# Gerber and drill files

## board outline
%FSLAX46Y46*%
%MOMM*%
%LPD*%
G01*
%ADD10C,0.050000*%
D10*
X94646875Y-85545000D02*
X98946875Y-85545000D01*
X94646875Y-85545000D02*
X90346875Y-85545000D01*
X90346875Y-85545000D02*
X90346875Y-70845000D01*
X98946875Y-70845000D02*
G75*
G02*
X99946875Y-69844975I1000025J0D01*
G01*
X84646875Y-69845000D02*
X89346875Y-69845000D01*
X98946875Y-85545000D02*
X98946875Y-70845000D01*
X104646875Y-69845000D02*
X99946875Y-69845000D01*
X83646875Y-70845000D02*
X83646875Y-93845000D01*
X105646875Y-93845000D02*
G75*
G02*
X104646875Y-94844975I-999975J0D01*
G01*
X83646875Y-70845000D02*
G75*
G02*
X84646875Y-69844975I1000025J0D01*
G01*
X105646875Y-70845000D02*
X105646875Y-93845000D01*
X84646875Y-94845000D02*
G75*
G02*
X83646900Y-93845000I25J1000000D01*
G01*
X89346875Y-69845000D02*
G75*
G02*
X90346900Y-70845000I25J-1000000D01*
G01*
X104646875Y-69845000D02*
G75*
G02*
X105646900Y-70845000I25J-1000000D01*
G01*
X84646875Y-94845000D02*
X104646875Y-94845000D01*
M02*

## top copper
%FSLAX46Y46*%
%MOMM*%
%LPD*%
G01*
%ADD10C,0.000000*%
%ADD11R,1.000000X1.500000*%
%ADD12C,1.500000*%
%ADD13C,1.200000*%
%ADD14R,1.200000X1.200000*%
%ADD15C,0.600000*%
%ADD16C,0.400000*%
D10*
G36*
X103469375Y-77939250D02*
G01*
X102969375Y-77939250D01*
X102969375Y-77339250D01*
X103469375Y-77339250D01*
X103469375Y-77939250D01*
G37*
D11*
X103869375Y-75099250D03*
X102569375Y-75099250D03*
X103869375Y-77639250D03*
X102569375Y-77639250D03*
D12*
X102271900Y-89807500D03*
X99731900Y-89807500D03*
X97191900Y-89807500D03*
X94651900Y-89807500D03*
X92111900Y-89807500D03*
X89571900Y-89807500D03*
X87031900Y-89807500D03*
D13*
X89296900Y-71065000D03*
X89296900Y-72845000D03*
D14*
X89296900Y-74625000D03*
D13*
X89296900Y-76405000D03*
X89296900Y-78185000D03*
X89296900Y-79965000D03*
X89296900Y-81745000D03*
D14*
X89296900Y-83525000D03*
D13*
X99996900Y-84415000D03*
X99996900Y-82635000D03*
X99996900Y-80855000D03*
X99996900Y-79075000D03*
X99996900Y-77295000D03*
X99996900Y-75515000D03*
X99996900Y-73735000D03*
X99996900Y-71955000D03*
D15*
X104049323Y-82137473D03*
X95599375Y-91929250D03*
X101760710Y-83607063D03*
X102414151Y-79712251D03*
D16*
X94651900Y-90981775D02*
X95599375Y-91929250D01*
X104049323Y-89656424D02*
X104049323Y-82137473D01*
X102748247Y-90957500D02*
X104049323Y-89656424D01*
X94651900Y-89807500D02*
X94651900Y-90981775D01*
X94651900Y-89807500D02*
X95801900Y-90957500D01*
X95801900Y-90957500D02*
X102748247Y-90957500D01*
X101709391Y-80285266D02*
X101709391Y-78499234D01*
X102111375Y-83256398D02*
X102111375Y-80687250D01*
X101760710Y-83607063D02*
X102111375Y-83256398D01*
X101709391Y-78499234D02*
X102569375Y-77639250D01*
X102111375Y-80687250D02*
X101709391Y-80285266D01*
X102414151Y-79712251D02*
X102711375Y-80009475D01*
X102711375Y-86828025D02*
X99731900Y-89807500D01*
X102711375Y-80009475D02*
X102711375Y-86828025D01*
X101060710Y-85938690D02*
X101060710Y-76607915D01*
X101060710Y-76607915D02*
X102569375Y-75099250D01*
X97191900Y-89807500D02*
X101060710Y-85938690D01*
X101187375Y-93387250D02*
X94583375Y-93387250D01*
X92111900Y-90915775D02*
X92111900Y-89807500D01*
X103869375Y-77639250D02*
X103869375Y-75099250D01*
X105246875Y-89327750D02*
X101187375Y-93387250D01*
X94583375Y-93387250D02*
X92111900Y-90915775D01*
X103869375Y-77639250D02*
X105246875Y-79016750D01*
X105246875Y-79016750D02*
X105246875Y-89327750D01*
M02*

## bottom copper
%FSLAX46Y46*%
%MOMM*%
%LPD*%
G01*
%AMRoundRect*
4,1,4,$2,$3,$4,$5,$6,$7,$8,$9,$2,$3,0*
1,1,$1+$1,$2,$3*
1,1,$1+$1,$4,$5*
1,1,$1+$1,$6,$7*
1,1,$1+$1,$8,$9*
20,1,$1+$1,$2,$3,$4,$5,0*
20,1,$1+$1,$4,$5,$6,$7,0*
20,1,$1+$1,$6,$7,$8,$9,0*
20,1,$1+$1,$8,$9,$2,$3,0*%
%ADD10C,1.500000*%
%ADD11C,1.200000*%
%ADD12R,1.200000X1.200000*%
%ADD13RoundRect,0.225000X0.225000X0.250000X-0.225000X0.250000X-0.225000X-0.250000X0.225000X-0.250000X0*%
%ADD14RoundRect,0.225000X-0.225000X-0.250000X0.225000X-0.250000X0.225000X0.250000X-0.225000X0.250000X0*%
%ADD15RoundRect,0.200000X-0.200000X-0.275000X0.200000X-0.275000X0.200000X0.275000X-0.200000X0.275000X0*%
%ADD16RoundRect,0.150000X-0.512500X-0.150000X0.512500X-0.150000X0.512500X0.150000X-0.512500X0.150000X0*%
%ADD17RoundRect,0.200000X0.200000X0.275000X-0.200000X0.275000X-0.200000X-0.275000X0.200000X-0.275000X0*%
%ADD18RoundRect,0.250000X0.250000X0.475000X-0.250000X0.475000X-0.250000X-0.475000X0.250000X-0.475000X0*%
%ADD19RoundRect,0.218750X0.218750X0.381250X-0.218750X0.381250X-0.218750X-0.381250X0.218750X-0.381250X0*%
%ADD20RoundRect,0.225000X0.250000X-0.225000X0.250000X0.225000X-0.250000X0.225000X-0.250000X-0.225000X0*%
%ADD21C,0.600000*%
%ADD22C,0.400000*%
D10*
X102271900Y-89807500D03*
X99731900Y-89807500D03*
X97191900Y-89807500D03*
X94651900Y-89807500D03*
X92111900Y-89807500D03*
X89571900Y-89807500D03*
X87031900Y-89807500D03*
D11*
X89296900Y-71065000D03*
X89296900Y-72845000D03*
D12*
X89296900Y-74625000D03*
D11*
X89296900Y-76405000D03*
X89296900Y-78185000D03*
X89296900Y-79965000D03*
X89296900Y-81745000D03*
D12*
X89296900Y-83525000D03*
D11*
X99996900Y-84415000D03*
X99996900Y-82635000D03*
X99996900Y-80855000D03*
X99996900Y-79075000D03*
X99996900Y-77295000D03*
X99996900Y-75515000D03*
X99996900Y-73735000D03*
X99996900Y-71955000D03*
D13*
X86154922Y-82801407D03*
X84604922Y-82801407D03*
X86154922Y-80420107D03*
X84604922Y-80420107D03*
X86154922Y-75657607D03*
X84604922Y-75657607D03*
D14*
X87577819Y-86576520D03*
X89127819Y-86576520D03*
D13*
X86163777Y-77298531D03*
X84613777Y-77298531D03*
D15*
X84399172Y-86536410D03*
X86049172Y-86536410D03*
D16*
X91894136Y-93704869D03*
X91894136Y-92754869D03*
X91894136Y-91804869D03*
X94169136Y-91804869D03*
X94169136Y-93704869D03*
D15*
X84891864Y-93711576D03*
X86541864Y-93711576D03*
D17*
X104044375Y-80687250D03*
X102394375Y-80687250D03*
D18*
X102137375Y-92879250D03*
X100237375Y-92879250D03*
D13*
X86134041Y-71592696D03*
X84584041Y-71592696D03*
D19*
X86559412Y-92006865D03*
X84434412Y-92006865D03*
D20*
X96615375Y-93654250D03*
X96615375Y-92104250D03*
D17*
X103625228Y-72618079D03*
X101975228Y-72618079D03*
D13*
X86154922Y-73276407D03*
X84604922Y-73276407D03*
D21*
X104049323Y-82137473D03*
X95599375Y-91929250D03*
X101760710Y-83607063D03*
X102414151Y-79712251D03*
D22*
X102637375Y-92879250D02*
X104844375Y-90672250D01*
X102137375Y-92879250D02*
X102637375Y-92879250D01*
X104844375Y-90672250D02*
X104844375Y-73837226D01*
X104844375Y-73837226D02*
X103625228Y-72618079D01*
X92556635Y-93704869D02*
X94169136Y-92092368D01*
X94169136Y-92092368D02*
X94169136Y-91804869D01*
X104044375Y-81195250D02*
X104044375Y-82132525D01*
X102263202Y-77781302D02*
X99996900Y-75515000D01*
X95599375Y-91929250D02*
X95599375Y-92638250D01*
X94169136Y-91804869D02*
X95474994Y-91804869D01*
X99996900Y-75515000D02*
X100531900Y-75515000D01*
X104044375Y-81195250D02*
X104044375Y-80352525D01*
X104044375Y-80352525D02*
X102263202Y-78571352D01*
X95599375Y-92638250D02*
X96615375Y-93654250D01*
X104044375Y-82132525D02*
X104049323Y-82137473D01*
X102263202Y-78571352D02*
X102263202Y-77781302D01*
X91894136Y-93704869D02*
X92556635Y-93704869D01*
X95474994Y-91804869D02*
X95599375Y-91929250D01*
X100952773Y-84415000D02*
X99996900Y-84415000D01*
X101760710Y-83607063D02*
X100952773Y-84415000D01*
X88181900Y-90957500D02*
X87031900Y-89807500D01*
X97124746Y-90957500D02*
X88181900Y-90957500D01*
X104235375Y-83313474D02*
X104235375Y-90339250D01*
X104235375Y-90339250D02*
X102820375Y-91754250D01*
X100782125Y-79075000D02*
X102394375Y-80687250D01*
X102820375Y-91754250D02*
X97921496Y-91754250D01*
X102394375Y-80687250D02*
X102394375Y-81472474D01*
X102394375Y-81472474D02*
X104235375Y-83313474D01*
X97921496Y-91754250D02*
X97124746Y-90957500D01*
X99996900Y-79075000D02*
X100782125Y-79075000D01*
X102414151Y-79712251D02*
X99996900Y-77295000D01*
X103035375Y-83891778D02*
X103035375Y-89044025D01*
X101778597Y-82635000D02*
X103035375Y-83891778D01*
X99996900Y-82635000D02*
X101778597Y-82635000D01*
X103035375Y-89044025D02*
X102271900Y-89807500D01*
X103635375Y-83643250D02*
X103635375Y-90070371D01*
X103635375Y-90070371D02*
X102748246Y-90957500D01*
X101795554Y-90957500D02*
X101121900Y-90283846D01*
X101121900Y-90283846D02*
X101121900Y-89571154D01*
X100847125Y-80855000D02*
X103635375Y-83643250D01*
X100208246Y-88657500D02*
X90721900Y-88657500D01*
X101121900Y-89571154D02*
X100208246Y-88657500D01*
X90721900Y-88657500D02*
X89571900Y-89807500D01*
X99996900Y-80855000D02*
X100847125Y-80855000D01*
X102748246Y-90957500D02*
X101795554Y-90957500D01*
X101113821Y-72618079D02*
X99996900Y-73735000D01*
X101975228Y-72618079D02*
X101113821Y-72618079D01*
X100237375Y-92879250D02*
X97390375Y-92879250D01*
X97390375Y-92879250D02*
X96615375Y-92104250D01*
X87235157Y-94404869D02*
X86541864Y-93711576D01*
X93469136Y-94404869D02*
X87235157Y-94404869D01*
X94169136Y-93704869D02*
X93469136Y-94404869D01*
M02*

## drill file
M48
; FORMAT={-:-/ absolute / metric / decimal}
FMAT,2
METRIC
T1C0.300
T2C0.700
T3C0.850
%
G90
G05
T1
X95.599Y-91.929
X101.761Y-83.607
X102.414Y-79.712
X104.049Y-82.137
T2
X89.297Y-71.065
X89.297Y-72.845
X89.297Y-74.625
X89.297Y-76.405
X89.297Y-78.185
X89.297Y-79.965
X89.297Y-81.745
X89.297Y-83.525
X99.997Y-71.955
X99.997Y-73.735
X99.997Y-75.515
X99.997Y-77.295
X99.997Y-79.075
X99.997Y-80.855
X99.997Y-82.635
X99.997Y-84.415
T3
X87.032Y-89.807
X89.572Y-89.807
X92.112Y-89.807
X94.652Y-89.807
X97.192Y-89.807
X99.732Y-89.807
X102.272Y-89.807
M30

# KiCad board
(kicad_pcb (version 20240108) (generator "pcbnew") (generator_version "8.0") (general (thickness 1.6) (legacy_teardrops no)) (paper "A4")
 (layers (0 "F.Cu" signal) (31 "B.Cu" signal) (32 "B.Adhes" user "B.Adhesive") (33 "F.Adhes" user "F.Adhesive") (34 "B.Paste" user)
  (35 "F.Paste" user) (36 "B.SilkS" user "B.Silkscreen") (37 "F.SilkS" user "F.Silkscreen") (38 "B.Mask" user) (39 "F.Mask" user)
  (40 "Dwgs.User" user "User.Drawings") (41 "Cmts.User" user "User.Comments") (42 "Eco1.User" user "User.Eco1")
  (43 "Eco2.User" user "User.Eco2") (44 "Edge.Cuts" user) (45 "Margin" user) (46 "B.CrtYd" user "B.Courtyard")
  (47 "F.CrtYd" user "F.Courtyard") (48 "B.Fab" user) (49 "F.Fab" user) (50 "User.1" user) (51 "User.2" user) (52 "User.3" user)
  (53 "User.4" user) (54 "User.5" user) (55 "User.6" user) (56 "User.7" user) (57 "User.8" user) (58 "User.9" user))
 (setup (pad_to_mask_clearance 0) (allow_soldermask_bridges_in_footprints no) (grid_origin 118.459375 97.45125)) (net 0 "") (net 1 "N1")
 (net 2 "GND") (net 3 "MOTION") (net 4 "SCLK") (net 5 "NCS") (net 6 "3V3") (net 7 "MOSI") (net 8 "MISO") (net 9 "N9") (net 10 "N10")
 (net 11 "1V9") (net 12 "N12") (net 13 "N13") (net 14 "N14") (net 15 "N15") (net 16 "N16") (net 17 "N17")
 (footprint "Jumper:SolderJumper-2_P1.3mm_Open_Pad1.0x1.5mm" (layer "F.Cu") (at 103.219375 75.09925 180)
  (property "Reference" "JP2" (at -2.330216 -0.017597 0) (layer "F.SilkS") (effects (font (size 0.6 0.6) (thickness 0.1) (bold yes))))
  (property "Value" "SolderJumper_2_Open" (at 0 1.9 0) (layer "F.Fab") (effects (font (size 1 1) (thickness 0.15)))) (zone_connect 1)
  (pad "1" smd rect (at -0.65 0 180) (size 1 1.5) (layers "F.Cu" "F.Mask") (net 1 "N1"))
  (pad "2" smd rect (at 0.65 0 180) (size 1 1.5) (layers "F.Cu" "F.Mask") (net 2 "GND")))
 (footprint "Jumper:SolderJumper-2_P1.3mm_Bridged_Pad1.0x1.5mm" (layer "F.Cu") (at 103.219375 77.63925 180)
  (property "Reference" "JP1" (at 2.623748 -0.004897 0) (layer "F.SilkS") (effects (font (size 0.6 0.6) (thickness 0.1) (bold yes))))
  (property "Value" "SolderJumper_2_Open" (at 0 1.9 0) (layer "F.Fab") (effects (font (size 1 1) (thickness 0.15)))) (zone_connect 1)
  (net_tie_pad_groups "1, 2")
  (fp_poly (pts (xy -0.25 -0.3) (xy 0.25 -0.3) (xy 0.25 0.3) (xy -0.25 0.3)) (stroke (width 0) (type solid)) (fill solid) (layer "F.Cu"))
  (pad "1" smd rect (at -0.65 0 180) (size 1 1.5) (layers "F.Cu" "F.Mask") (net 1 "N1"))
  (pad "2" smd rect (at 0.65 0 180) (size 1 1.5) (layers "F.Cu" "F.Mask") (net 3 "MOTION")))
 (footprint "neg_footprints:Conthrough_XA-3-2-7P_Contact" (layer "F.Cu") (at 102.2719 89.8075 -90)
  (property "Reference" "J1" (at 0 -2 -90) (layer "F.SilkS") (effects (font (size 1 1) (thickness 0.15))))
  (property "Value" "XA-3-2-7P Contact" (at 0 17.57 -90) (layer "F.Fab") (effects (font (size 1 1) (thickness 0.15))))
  (pad "1" thru_hole circle (at 0 0 270) (size 1.5 1.5) (drill 0.85) (layers "*.Cu" "*.Mask") (remove_unused_layers no) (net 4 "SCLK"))
  (pad "2" thru_hole circle (at 0 2.54 270) (size 1.5 1.5) (drill 0.85) (layers "*.Cu" "*.Mask") (remove_unused_layers no) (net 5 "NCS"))
  (pad "3" thru_hole circle (at 0 5.08 270) (size 1.5 1.5) (drill 0.85) (layers "*.Cu" "*.Mask") (remove_unused_layers no) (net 2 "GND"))
  (pad "4" thru_hole circle (at 0 7.62 270) (size 1.5 1.5) (drill 0.85) (layers "*.Cu" "*.Mask") (remove_unused_layers no) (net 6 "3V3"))
  (pad "5" thru_hole circle (at 0 10.16 270) (size 1.5 1.5) (drill 0.85) (layers "*.Cu" "*.Mask") (remove_unused_layers no) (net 1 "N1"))
  (pad "6" thru_hole circle (at 0 12.7 270) (size 1.5 1.5) (drill 0.85) (layers "*.Cu" "*.Mask") (remove_unused_layers no) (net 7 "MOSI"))
  (pad "7" thru_hole circle (at 0 15.24 270) (size 1.5 1.5) (drill 0.85) (layers "*.Cu" "*.Mask") (remove_unused_layers no) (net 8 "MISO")))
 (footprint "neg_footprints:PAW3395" (layer "F.Cu") (at 94.6469 76.405)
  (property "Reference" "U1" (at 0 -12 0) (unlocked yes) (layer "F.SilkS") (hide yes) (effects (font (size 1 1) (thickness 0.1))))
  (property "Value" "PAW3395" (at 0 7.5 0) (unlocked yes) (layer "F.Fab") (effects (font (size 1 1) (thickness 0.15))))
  (pad "1" thru_hole circle (at -5.35 -5.34) (size 1.2 1.2) (drill 0.7) (layers "*.Cu" "*.Mask") (remove_unused_layers no) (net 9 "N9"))
  (pad "2" thru_hole circle (at -5.35 -3.56) (size 1.2 1.2) (drill 0.7) (layers "*.Cu" "*.Mask") (remove_unused_layers no) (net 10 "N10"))
  (pad "3" thru_hole rect (at -5.35 -1.78) (size 1.2 1.2) (drill 0.7) (layers "*.Cu" "*.Mask") (remove_unused_layers no) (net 2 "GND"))
  (pad "4" thru_hole circle (at -5.35 0) (size 1.2 1.2) (drill 0.7) (layers "*.Cu" "*.Mask") (remove_unused_layers no) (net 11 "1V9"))
  (pad "5" thru_hole circle (at -5.35 1.78) (size 1.2 1.2) (drill 0.7) (layers "*.Cu" "*.Mask") (remove_unused_layers no) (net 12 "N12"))
  (pad "6" thru_hole circle (at -5.35 3.56) (size 1.2 1.2) (drill 0.7) (layers "*.Cu" "*.Mask") (remove_unused_layers no) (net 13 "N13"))
  (pad "7" thru_hole circle (at -5.35 5.34) (size 1.2 1.2) (drill 0.7) (layers "*.Cu" "*.Mask") (remove_unused_layers no) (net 6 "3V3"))
  (pad "8" thru_hole rect (at -5.35 7.12) (size 1.2 1.2) (drill 0.7) (layers "*.Cu" "*.Mask") (remove_unused_layers no) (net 2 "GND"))
  (pad "9" thru_hole circle (at 5.35 8.01) (size 1.2 1.2) (drill 0.7) (layers "*.Cu" "*.Mask") (remove_unused_layers no) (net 3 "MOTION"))
  (pad "10" thru_hole circle (at 5.35 6.23) (size 1.2 1.2) (drill 0.7) (layers "*.Cu" "*.Mask") (remove_unused_layers no) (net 4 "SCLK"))
  (pad "11" thru_hole circle (at 5.35 4.45) (size 1.2 1.2) (drill 0.7) (layers "*.Cu" "*.Mask") (remove_unused_layers no) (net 7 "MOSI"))
  (pad "12" thru_hole circle (at 5.35 2.67) (size 1.2 1.2) (drill 0.7) (layers "*.Cu" "*.Mask") (remove_unused_layers no) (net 8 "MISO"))
  (pad "13" thru_hole circle (at 5.35 0.89) (size 1.2 1.2) (drill 0.7) (layers "*.Cu" "*.Mask") (remove_unused_layers no) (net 5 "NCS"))
  (pad "14" thru_hole circle (at 5.35 -0.89) (size 1.2 1.2) (drill 0.7) (layers "*.Cu" "*.Mask") (remove_unused_layers no) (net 6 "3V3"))
  (pad "15" thru_hole circle (at 5.35 -2.67) (size 1.2 1.2) (drill 0.7) (layers "*.Cu" "*.Mask") (remove_unused_layers no) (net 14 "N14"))
  (pad "16" thru_hole circle (at 5.35 -4.45) (size 1.2 1.2) (drill 0.7) (layers "*.Cu" "*.Mask") (remove_unused_layers no) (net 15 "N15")))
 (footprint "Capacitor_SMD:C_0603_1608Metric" (layer "B.Cu") (at 85.379922 82.801407 180)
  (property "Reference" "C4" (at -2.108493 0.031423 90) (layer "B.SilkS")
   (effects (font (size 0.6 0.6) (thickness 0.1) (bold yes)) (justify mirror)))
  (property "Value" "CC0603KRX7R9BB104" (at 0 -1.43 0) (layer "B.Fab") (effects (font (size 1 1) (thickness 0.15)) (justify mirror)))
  (pad "1" smd roundrect (at -0.775 0 180) (size 0.9 0.95) (layers "B.Cu" "B.Paste" "B.Mask") (roundrect_rratio 0.25) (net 6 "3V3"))
  (pad "2" smd roundrect (at 0.775 0 180) (size 0.9 0.95) (layers "B.Cu" "B.Paste" "B.Mask") (roundrect_rratio 0.25) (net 2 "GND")))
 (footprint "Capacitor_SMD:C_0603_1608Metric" (layer "B.Cu") (at 85.379922 80.420107 180)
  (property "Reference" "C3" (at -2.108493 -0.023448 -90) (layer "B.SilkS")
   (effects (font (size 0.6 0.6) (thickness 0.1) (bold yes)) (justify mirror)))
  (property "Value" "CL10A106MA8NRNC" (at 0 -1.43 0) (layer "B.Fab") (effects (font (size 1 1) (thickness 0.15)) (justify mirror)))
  (pad "1" smd roundrect (at -0.775 0 180) (size 0.9 0.95) (layers "B.Cu" "B.Paste" "B.Mask") (roundrect_rratio 0.25) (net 6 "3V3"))
  (pad "2" smd roundrect (at 0.775 0 180) (size 0.9 0.95) (layers "B.Cu" "B.Paste" "B.Mask") (roundrect_rratio 0.25) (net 2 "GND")))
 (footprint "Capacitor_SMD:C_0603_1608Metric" (layer "B.Cu") (at 85.379922 75.657607 180)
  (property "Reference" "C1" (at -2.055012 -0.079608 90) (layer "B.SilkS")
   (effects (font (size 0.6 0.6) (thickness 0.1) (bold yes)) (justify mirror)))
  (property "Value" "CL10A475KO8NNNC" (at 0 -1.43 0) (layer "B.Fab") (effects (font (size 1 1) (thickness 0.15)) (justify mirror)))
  (pad "1" smd roundrect (at -0.775 0 180) (size 0.9 0.95) (layers "B.Cu" "B.Paste" "B.Mask") (roundrect_rratio 0.25) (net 12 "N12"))
  (pad "2" smd roundrect (at 0.775 0 180) (size 0.9 0.95) (layers "B.Cu" "B.Paste" "B.Mask") (roundrect_rratio 0.25) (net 2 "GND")))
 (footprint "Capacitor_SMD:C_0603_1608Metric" (layer "B.Cu") (at 88.352819 86.57652)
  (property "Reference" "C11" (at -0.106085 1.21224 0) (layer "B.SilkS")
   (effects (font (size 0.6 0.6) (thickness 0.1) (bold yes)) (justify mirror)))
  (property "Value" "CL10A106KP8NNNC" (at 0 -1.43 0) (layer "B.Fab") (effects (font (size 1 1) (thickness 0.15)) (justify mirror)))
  (pad "1" smd roundrect (at -0.775 0) (size 0.9 0.95) (layers "B.Cu" "B.Paste" "B.Mask") (roundrect_rratio 0.25) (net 11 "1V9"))
  (pad "2" smd roundrect (at 0.775 0) (size 0.9 0.95) (layers "B.Cu" "B.Paste" "B.Mask") (roundrect_rratio 0.25) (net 2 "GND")))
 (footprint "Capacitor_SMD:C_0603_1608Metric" (layer "B.Cu") (at 85.388777 77.298531 180)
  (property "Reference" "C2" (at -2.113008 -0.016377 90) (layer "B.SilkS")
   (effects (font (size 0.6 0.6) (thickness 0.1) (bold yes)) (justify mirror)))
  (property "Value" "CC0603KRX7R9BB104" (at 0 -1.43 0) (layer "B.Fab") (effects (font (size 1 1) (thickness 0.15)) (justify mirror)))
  (pad "1" smd roundrect (at -0.775 0 180) (size 0.9 0.95) (layers "B.Cu" "B.Paste" "B.Mask") (roundrect_rratio 0.25) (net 12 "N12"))
  (pad "2" smd roundrect (at 0.775 0 180) (size 0.9 0.95) (layers "B.Cu" "B.Paste" "B.Mask") (roundrect_rratio 0.25) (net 2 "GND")))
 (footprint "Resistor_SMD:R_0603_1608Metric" (layer "B.Cu") (at 85.224172 86.53641)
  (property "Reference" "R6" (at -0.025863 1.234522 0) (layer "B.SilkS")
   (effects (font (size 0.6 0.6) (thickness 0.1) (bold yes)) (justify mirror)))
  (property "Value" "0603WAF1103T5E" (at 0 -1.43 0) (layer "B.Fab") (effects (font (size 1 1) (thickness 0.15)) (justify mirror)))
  (pad "1" smd roundrect (at -0.825 0) (size 0.8 0.95) (layers "B.Cu" "B.Paste" "B.Mask") (roundrect_rratio 0.25) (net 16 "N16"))
  (pad "2" smd roundrect (at 0.825 0) (size 0.8 0.95) (layers "B.Cu" "B.Paste" "B.Mask") (roundrect_rratio 0.25) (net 2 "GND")))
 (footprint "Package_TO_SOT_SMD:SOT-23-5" (layer "B.Cu") (at 93.031636 92.754869)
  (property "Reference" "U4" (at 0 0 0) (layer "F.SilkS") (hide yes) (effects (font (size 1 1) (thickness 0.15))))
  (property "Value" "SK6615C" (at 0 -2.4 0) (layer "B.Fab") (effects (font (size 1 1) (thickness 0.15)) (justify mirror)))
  (pad "1" smd roundrect (at -1.1375 0.95) (size 1.325 0.6) (layers "B.Cu" "B.Paste" "B.Mask") (roundrect_rratio 0.25) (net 6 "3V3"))
  (pad "2" smd roundrect (at -1.1375 0) (size 1.325 0.6) (layers "B.Cu" "B.Paste" "B.Mask") (roundrect_rratio 0.25) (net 2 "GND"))
  (pad "3" smd roundrect (at -1.1375 -0.95) (size 1.325 0.6) (layers "B.Cu" "B.Paste" "B.Mask") (roundrect_rratio 0.25) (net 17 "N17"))
  (pad "4" smd roundrect (at 1.1375 -0.95) (size 1.325 0.6) (layers "B.Cu" "B.Paste" "B.Mask") (roundrect_rratio 0.25) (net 6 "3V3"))
  (pad "5" smd roundrect (at 1.1375 0.95) (size 1.325 0.6) (layers "B.Cu" "B.Paste" "B.Mask") (roundrect_rratio 0.25) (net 16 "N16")))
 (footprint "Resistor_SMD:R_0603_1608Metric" (layer "B.Cu") (at 85.716864 93.711576)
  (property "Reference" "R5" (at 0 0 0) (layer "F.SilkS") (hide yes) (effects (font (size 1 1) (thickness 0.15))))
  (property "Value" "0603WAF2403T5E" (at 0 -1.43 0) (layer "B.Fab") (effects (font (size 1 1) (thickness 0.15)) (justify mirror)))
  (pad "1" smd roundrect (at -0.825 0) (size 0.8 0.95) (layers "B.Cu" "B.Paste" "B.Mask") (roundrect_rratio 0.25) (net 11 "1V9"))
  (pad "2" smd roundrect (at 0.825 0) (size 0.8 0.95) (layers "B.Cu" "B.Paste" "B.Mask") (roundrect_rratio 0.25) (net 16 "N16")))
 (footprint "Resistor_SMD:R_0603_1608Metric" (layer "B.Cu") (at 103.219375 80.68725 180)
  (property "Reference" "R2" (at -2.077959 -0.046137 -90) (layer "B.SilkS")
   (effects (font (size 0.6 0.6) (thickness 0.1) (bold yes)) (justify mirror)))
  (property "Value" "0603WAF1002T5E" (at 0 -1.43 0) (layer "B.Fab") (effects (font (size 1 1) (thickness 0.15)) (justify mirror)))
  (pad "1" smd roundrect (at -0.825 0 180) (size 0.8 0.95) (layers "B.Cu" "B.Paste" "B.Mask") (roundrect_rratio 0.25) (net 6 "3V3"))
  (pad "2" smd roundrect (at 0.825 0 180) (size 0.8 0.95) (layers "B.Cu" "B.Paste" "B.Mask") (roundrect_rratio 0.25) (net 8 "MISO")))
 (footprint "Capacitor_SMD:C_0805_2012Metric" (layer "B.Cu") (at 101.187375 92.87925 180)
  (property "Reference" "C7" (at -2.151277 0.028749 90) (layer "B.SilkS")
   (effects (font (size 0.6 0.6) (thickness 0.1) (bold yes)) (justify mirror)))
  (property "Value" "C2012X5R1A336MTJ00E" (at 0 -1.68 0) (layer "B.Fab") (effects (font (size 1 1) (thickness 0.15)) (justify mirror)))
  (pad "1" smd roundrect (at -0.95 0 180) (size 1 1.45) (layers "B.Cu" "B.Paste" "B.Mask") (roundrect_rratio 0.25) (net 11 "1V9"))
  (pad "2" smd roundrect (at 0.95 0 180) (size 1 1.45) (layers "B.Cu" "B.Paste" "B.Mask") (roundrect_rratio 0.25) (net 2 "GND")))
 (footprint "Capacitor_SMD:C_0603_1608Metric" (layer "B.Cu") (at 85.359041 71.592696 180)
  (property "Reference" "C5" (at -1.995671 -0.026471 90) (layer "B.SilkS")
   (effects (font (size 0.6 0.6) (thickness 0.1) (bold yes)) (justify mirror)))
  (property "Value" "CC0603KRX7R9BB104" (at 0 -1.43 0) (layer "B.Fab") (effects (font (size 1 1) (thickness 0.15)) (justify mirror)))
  (pad "1" smd roundrect (at -0.775 0 180) (size 0.9 0.95) (layers "B.Cu" "B.Paste" "B.Mask") (roundrect_rratio 0.25) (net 11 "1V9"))
  (pad "2" smd roundrect (at 0.775 0 180) (size 0.9 0.95) (layers "B.Cu" "B.Paste" "B.Mask") (roundrect_rratio 0.25) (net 2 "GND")))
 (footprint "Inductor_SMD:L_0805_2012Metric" (layer "B.Cu") (at 85.496912 92.006865 180)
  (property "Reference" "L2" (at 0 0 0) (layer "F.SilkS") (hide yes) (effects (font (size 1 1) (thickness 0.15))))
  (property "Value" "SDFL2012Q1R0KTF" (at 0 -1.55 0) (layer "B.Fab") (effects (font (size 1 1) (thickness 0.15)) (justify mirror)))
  (pad "1" smd roundrect (at -1.0625 0 180) (size 0.875 1.2) (layers "B.Cu" "B.Paste" "B.Mask") (roundrect_rratio 0.25) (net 17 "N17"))
  (pad "2" smd roundrect (at 1.0625 0 180) (size 0.875 1.2) (layers "B.Cu" "B.Paste" "B.Mask") (roundrect_rratio 0.25) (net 11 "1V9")))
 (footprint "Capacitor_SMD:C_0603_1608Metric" (layer "B.Cu") (at 96.615375 92.87925 90)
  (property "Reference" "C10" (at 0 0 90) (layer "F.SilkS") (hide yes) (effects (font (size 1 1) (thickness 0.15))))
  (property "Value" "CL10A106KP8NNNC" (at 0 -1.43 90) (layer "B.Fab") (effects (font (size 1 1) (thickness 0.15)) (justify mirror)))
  (pad "1" smd roundrect (at -0.775 0 90) (size 0.9 0.95) (layers "B.Cu" "B.Paste" "B.Mask") (roundrect_rratio 0.25) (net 6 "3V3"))
  (pad "2" smd roundrect (at 0.775 0 90) (size 0.9 0.95) (layers "B.Cu" "B.Paste" "B.Mask") (roundrect_rratio 0.25) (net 2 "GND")))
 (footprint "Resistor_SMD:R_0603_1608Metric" (layer "B.Cu") (at 102.800228 72.618079 180)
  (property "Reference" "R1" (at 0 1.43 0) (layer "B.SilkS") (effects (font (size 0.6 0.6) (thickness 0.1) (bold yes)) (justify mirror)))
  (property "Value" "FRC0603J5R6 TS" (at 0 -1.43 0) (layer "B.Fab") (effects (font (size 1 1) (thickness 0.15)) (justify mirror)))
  (pad "1" smd roundrect (at -0.825 0 180) (size 0.8 0.95) (layers "B.Cu" "B.Paste" "B.Mask") (roundrect_rratio 0.25) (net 11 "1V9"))
  (pad "2" smd roundrect (at 0.825 0 180) (size 0.8 0.95) (layers "B.Cu" "B.Paste" "B.Mask") (roundrect_rratio 0.25) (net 14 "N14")))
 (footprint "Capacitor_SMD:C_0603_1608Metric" (layer "B.Cu") (at 85.379922 73.276407 180)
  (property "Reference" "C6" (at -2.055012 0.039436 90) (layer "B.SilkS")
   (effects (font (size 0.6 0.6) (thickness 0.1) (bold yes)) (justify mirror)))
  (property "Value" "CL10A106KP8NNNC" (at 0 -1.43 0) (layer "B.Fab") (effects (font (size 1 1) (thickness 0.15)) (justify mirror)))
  (pad "1" smd roundrect (at -0.775 0 180) (size 0.9 0.95) (layers "B.Cu" "B.Paste" "B.Mask") (roundrect_rratio 0.25) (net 11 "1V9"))
  (pad "2" smd roundrect (at 0.775 0 180) (size 0.9 0.95) (layers "B.Cu" "B.Paste" "B.Mask") (roundrect_rratio 0.25) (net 2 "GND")))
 (gr_line (start 94.646875 85.545) (end 98.946875 85.545) (stroke (width 0.05) (type solid)) (layer "Edge.Cuts"))
 (gr_line (start 94.646875 85.545) (end 90.346875 85.545) (stroke (width 0.05) (type solid)) (layer "Edge.Cuts"))
 (gr_line (start 90.346875 85.545) (end 90.346875 70.845) (stroke (width 0.05) (type solid)) (layer "Edge.Cuts"))
 (gr_arc (start 98.946875 70.845) (mid 99.239768 70.137893) (end 99.946875 69.845) (stroke (width 0.05) (type default)) (layer "Edge.Cuts"))
 (gr_line (start 84.646875 69.845) (end 89.346875 69.845) (stroke (width 0.05) (type solid)) (layer "Edge.Cuts"))
 (gr_line (start 98.946875 85.545) (end 98.946875 70.845) (stroke (width 0.05) (type solid)) (layer "Edge.Cuts"))
 (gr_line (start 104.646875 69.845) (end 99.946875 69.845) (stroke (width 0.05) (type solid)) (layer "Edge.Cuts"))
 (gr_line (start 83.646875 70.845) (end 83.646875 93.845) (stroke (width 0.05) (type solid)) (layer "Edge.Cuts"))
 (gr_arc (start 105.646875 93.845) (mid 105.35398 94.552098) (end 104.646875 94.845) (stroke (width 0.05) (type default))
  (layer "Edge.Cuts"))
 (gr_arc (start 83.646875 70.845) (mid 83.939768 70.137893) (end 84.646875 69.845) (stroke (width 0.05) (type default)) (layer "Edge.Cuts"))
 (gr_line (start 105.646875 70.845) (end 105.646875 93.845) (stroke (width 0.05) (type solid)) (layer "Edge.Cuts"))
 (gr_arc (start 84.646875 94.845) (mid 83.939768 94.552107) (end 83.646875 93.845) (stroke (width 0.05) (type default)) (layer "Edge.Cuts"))
 (gr_arc (start 89.346875 69.845) (mid 90.053998 70.137884) (end 90.346875 70.845) (stroke (width 0.05) (type default)) (layer "Edge.Cuts"))
 (gr_arc (start 104.646875 69.845) (mid 105.353998 70.137884) (end 105.646875 70.845) (stroke (width 0.05) (type default))
  (layer "Edge.Cuts"))
 (gr_line (start 84.646875 94.845) (end 104.646875 94.845) (stroke (width 0.05) (type solid)) (layer "Edge.Cuts"))
 (segment (start 102.637375 92.87925) (end 104.844375 90.67225) (width 0.4) (layer "B.Cu") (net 11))
 (segment (start 102.137375 92.87925) (end 102.637375 92.87925) (width 0.4) (layer "B.Cu") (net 11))
 (segment (start 104.844375 90.67225) (end 104.844375 73.837226) (width 0.4) (layer "B.Cu") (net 11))
 (segment (start 104.844375 73.837226) (end 103.625228 72.618079) (width 0.4) (layer "B.Cu") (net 11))
 (segment (start 94.6519 90.981775) (end 95.599375 91.92925) (width 0.4) (layer "F.Cu") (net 6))
 (segment (start 104.049323 89.656424) (end 104.049323 82.137473) (width 0.4) (layer "F.Cu") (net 6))
 (segment (start 102.748247 90.9575) (end 104.049323 89.656424) (width 0.4) (layer "F.Cu") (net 6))
 (segment (start 94.6519 89.8075) (end 94.6519 90.981775) (width 0.4) (layer "F.Cu") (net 6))
 (segment (start 94.6519 89.8075) (end 95.8019 90.9575) (width 0.4) (layer "F.Cu") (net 6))
 (segment (start 95.8019 90.9575) (end 102.748247 90.9575) (width 0.4) (layer "F.Cu") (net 6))
 (via (at 104.049323 82.137473) (size 0.6) (drill 0.3) (layers "F.Cu" "B.Cu") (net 6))
 (via (at 95.599375 91.92925) (size 0.6) (drill 0.3) (layers "F.Cu" "B.Cu") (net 6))
 (segment (start 92.556635 93.704869) (end 94.169136 92.092368) (width 0.4) (layer "B.Cu") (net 6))
 (segment (start 94.169136 92.092368) (end 94.169136 91.804869) (width 0.4) (layer "B.Cu") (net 6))
 (segment (start 104.044375 81.19525) (end 104.044375 82.132525) (width 0.4) (layer "B.Cu") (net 6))
 (segment (start 102.263202 77.781302) (end 99.9969 75.515) (width 0.4) (layer "B.Cu") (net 6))
 (segment (start 95.599375 91.92925) (end 95.599375 92.63825) (width 0.4) (layer "B.Cu") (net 6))
 (segment (start 94.169136 91.804869) (end 95.474994 91.804869) (width 0.4) (layer "B.Cu") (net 6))
 (segment (start 99.9969 75.515) (end 100.5319 75.515) (width 0.4) (layer "B.Cu") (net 6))
 (segment (start 104.044375 81.19525) (end 104.044375 80.352525) (width 0.4) (layer "B.Cu") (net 6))
 (segment (start 104.044375 80.352525) (end 102.263202 78.571352) (width 0.4) (layer "B.Cu") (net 6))
 (segment (start 95.599375 92.63825) (end 96.615375 93.65425) (width 0.4) (layer "B.Cu") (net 6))
 (segment (start 104.044375 82.132525) (end 104.049323 82.137473) (width 0.4) (layer "B.Cu") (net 6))
 (segment (start 102.263202 78.571352) (end 102.263202 77.781302) (width 0.4) (layer "B.Cu") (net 6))
 (segment (start 91.894136 93.704869) (end 92.556635 93.704869) (width 0.4) (layer "B.Cu") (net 6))
 (segment (start 95.474994 91.804869) (end 95.599375 91.92925) (width 0.4) (layer "B.Cu") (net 6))
 (segment (start 101.709391 80.285266) (end 101.709391 78.499234) (width 0.4) (layer "F.Cu") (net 3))
 (segment (start 102.111375 83.256398) (end 102.111375 80.68725) (width 0.4) (layer "F.Cu") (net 3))
 (segment (start 101.76071 83.607063) (end 102.111375 83.256398) (width 0.4) (layer "F.Cu") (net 3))
 (segment (start 101.709391 78.499234) (end 102.569375 77.63925) (width 0.4) (layer "F.Cu") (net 3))
 (segment (start 102.111375 80.68725) (end 101.709391 80.285266) (width 0.4) (layer "F.Cu") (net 3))
 (via (at 101.76071 83.607063) (size 0.6) (drill 0.3) (layers "F.Cu" "B.Cu") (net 3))
 (segment (start 100.952773 84.415) (end 99.9969 84.415) (width 0.4) (layer "B.Cu") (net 3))
 (segment (start 101.76071 83.607063) (end 100.952773 84.415) (width 0.4) (layer "B.Cu") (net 3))
 (segment (start 88.1819 90.9575) (end 87.0319 89.8075) (width 0.4) (layer "B.Cu") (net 8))
 (segment (start 97.124746 90.9575) (end 88.1819 90.9575) (width 0.4) (layer "B.Cu") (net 8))
 (segment (start 104.235375 83.313474) (end 104.235375 90.33925) (width 0.4) (layer "B.Cu") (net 8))
 (segment (start 104.235375 90.33925) (end 102.820375 91.75425) (width 0.4) (layer "B.Cu") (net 8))
 (segment (start 100.782125 79.075) (end 102.394375 80.68725) (width 0.4) (layer "B.Cu") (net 8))
 (segment (start 102.820375 91.75425) (end 97.921496 91.75425) (width 0.4) (layer "B.Cu") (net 8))
 (segment (start 102.394375 80.68725) (end 102.394375 81.472474) (width 0.4) (layer "B.Cu") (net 8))
 (segment (start 102.394375 81.472474) (end 104.235375 83.313474) (width 0.4) (layer "B.Cu") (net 8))
 (segment (start 97.921496 91.75425) (end 97.124746 90.9575) (width 0.4) (layer "B.Cu") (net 8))
 (segment (start 99.9969 79.075) (end 100.782125 79.075) (width 0.4) (layer "B.Cu") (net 8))
 (segment (start 102.414151 79.712251) (end 102.711375 80.009475) (width 0.4) (layer "F.Cu") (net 5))
 (segment (start 102.711375 86.828025) (end 99.7319 89.8075) (width 0.4) (layer "F.Cu") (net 5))
 (segment (start 102.711375 80.009475) (end 102.711375 86.828025) (width 0.4) (layer "F.Cu") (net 5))
 (via (at 102.414151 79.712251) (size 0.6) (drill 0.3) (layers "F.Cu" "B.Cu") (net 5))
 (segment (start 102.414151 79.712251) (end 99.9969 77.295) (width 0.4) (layer "B.Cu") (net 5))
 (segment (start 103.035375 83.891778) (end 103.035375 89.044025) (width 0.4) (layer "B.Cu") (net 4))
 (segment (start 101.778597 82.635) (end 103.035375 83.891778) (width 0.4) (layer "B.Cu") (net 4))
 (segment (start 99.9969 82.635) (end 101.778597 82.635) (width 0.4) (layer "B.Cu") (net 4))
 (segment (start 103.035375 89.044025) (end 102.2719 89.8075) (width 0.4) (layer "B.Cu") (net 4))
 (segment (start 103.635375 83.64325) (end 103.635375 90.070371) (width 0.4) (layer "B.Cu") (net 7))
 (segment (start 103.635375 90.070371) (end 102.748246 90.9575) (width 0.4) (layer "B.Cu") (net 7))
 (segment (start 101.795554 90.9575) (end 101.1219 90.283846) (width 0.4) (layer "B.Cu") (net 7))
 (segment (start 101.1219 90.283846) (end 101.1219 89.571154) (width 0.4) (layer "B.Cu") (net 7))
 (segment (start 100.847125 80.855) (end 103.635375 83.64325) (width 0.4) (layer "B.Cu") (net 7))
 (segment (start 100.208246 88.6575) (end 90.7219 88.6575) (width 0.4) (layer "B.Cu") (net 7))
 (segment (start 101.1219 89.571154) (end 100.208246 88.6575) (width 0.4) (layer "B.Cu") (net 7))
 (segment (start 90.7219 88.6575) (end 89.5719 89.8075) (width 0.4) (layer "B.Cu") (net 7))
 (segment (start 99.9969 80.855) (end 100.847125 80.855) (width 0.4) (layer "B.Cu") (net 7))
 (segment (start 102.748246 90.9575) (end 101.795554 90.9575) (width 0.4) (layer "B.Cu") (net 7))
 (segment (start 101.113821 72.618079) (end 99.9969 73.735) (width 0.4) (layer "B.Cu") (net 14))
 (segment (start 101.975228 72.618079) (end 101.113821 72.618079) (width 0.4) (layer "B.Cu") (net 14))
 (segment (start 101.06071 85.93869) (end 101.06071 76.607915) (width 0.4) (layer "F.Cu") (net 2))
 (segment (start 101.06071 76.607915) (end 102.569375 75.09925) (width 0.4) (layer "F.Cu") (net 2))
 (segment (start 97.1919 89.8075) (end 101.06071 85.93869) (width 0.4) (layer "F.Cu") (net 2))
 (segment (start 100.237375 92.87925) (end 97.390375 92.87925) (width 0.4) (layer "B.Cu") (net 2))
 (segment (start 97.390375 92.87925) (end 96.615375 92.10425) (width 0.4) (layer "B.Cu") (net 2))
 (segment (start 87.235157 94.404869) (end 86.541864 93.711576) (width 0.4) (layer "B.Cu") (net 16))
 (segment (start 93.469136 94.404869) (end 87.235157 94.404869) (width 0.4) (layer "B.Cu") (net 16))
 (segment (start 94.169136 93.704869) (end 93.469136 94.404869) (width 0.4) (layer "B.Cu") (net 16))
 (segment (start 101.187375 93.38725) (end 94.583375 93.38725) (width 0.4) (layer "F.Cu") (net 1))
 (segment (start 92.1119 90.915775) (end 92.1119 89.8075) (width 0.4) (layer "F.Cu") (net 1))
 (segment (start 103.869375 77.63925) (end 103.869375 75.09925) (width 0.4) (layer "F.Cu") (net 1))
 (segment (start 105.246875 89.32775) (end 101.187375 93.38725) (width 0.4) (layer "F.Cu") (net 1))
 (segment (start 94.583375 93.38725) (end 92.1119 90.915775) (width 0.4) (layer "F.Cu") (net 1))
 (segment (start 103.869375 77.63925) (end 105.246875 79.01675) (width 0.4) (layer "F.Cu") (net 1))
 (segment (start 105.246875 79.01675) (end 105.246875 89.32775) (width 0.4) (layer "F.Cu") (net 1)))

